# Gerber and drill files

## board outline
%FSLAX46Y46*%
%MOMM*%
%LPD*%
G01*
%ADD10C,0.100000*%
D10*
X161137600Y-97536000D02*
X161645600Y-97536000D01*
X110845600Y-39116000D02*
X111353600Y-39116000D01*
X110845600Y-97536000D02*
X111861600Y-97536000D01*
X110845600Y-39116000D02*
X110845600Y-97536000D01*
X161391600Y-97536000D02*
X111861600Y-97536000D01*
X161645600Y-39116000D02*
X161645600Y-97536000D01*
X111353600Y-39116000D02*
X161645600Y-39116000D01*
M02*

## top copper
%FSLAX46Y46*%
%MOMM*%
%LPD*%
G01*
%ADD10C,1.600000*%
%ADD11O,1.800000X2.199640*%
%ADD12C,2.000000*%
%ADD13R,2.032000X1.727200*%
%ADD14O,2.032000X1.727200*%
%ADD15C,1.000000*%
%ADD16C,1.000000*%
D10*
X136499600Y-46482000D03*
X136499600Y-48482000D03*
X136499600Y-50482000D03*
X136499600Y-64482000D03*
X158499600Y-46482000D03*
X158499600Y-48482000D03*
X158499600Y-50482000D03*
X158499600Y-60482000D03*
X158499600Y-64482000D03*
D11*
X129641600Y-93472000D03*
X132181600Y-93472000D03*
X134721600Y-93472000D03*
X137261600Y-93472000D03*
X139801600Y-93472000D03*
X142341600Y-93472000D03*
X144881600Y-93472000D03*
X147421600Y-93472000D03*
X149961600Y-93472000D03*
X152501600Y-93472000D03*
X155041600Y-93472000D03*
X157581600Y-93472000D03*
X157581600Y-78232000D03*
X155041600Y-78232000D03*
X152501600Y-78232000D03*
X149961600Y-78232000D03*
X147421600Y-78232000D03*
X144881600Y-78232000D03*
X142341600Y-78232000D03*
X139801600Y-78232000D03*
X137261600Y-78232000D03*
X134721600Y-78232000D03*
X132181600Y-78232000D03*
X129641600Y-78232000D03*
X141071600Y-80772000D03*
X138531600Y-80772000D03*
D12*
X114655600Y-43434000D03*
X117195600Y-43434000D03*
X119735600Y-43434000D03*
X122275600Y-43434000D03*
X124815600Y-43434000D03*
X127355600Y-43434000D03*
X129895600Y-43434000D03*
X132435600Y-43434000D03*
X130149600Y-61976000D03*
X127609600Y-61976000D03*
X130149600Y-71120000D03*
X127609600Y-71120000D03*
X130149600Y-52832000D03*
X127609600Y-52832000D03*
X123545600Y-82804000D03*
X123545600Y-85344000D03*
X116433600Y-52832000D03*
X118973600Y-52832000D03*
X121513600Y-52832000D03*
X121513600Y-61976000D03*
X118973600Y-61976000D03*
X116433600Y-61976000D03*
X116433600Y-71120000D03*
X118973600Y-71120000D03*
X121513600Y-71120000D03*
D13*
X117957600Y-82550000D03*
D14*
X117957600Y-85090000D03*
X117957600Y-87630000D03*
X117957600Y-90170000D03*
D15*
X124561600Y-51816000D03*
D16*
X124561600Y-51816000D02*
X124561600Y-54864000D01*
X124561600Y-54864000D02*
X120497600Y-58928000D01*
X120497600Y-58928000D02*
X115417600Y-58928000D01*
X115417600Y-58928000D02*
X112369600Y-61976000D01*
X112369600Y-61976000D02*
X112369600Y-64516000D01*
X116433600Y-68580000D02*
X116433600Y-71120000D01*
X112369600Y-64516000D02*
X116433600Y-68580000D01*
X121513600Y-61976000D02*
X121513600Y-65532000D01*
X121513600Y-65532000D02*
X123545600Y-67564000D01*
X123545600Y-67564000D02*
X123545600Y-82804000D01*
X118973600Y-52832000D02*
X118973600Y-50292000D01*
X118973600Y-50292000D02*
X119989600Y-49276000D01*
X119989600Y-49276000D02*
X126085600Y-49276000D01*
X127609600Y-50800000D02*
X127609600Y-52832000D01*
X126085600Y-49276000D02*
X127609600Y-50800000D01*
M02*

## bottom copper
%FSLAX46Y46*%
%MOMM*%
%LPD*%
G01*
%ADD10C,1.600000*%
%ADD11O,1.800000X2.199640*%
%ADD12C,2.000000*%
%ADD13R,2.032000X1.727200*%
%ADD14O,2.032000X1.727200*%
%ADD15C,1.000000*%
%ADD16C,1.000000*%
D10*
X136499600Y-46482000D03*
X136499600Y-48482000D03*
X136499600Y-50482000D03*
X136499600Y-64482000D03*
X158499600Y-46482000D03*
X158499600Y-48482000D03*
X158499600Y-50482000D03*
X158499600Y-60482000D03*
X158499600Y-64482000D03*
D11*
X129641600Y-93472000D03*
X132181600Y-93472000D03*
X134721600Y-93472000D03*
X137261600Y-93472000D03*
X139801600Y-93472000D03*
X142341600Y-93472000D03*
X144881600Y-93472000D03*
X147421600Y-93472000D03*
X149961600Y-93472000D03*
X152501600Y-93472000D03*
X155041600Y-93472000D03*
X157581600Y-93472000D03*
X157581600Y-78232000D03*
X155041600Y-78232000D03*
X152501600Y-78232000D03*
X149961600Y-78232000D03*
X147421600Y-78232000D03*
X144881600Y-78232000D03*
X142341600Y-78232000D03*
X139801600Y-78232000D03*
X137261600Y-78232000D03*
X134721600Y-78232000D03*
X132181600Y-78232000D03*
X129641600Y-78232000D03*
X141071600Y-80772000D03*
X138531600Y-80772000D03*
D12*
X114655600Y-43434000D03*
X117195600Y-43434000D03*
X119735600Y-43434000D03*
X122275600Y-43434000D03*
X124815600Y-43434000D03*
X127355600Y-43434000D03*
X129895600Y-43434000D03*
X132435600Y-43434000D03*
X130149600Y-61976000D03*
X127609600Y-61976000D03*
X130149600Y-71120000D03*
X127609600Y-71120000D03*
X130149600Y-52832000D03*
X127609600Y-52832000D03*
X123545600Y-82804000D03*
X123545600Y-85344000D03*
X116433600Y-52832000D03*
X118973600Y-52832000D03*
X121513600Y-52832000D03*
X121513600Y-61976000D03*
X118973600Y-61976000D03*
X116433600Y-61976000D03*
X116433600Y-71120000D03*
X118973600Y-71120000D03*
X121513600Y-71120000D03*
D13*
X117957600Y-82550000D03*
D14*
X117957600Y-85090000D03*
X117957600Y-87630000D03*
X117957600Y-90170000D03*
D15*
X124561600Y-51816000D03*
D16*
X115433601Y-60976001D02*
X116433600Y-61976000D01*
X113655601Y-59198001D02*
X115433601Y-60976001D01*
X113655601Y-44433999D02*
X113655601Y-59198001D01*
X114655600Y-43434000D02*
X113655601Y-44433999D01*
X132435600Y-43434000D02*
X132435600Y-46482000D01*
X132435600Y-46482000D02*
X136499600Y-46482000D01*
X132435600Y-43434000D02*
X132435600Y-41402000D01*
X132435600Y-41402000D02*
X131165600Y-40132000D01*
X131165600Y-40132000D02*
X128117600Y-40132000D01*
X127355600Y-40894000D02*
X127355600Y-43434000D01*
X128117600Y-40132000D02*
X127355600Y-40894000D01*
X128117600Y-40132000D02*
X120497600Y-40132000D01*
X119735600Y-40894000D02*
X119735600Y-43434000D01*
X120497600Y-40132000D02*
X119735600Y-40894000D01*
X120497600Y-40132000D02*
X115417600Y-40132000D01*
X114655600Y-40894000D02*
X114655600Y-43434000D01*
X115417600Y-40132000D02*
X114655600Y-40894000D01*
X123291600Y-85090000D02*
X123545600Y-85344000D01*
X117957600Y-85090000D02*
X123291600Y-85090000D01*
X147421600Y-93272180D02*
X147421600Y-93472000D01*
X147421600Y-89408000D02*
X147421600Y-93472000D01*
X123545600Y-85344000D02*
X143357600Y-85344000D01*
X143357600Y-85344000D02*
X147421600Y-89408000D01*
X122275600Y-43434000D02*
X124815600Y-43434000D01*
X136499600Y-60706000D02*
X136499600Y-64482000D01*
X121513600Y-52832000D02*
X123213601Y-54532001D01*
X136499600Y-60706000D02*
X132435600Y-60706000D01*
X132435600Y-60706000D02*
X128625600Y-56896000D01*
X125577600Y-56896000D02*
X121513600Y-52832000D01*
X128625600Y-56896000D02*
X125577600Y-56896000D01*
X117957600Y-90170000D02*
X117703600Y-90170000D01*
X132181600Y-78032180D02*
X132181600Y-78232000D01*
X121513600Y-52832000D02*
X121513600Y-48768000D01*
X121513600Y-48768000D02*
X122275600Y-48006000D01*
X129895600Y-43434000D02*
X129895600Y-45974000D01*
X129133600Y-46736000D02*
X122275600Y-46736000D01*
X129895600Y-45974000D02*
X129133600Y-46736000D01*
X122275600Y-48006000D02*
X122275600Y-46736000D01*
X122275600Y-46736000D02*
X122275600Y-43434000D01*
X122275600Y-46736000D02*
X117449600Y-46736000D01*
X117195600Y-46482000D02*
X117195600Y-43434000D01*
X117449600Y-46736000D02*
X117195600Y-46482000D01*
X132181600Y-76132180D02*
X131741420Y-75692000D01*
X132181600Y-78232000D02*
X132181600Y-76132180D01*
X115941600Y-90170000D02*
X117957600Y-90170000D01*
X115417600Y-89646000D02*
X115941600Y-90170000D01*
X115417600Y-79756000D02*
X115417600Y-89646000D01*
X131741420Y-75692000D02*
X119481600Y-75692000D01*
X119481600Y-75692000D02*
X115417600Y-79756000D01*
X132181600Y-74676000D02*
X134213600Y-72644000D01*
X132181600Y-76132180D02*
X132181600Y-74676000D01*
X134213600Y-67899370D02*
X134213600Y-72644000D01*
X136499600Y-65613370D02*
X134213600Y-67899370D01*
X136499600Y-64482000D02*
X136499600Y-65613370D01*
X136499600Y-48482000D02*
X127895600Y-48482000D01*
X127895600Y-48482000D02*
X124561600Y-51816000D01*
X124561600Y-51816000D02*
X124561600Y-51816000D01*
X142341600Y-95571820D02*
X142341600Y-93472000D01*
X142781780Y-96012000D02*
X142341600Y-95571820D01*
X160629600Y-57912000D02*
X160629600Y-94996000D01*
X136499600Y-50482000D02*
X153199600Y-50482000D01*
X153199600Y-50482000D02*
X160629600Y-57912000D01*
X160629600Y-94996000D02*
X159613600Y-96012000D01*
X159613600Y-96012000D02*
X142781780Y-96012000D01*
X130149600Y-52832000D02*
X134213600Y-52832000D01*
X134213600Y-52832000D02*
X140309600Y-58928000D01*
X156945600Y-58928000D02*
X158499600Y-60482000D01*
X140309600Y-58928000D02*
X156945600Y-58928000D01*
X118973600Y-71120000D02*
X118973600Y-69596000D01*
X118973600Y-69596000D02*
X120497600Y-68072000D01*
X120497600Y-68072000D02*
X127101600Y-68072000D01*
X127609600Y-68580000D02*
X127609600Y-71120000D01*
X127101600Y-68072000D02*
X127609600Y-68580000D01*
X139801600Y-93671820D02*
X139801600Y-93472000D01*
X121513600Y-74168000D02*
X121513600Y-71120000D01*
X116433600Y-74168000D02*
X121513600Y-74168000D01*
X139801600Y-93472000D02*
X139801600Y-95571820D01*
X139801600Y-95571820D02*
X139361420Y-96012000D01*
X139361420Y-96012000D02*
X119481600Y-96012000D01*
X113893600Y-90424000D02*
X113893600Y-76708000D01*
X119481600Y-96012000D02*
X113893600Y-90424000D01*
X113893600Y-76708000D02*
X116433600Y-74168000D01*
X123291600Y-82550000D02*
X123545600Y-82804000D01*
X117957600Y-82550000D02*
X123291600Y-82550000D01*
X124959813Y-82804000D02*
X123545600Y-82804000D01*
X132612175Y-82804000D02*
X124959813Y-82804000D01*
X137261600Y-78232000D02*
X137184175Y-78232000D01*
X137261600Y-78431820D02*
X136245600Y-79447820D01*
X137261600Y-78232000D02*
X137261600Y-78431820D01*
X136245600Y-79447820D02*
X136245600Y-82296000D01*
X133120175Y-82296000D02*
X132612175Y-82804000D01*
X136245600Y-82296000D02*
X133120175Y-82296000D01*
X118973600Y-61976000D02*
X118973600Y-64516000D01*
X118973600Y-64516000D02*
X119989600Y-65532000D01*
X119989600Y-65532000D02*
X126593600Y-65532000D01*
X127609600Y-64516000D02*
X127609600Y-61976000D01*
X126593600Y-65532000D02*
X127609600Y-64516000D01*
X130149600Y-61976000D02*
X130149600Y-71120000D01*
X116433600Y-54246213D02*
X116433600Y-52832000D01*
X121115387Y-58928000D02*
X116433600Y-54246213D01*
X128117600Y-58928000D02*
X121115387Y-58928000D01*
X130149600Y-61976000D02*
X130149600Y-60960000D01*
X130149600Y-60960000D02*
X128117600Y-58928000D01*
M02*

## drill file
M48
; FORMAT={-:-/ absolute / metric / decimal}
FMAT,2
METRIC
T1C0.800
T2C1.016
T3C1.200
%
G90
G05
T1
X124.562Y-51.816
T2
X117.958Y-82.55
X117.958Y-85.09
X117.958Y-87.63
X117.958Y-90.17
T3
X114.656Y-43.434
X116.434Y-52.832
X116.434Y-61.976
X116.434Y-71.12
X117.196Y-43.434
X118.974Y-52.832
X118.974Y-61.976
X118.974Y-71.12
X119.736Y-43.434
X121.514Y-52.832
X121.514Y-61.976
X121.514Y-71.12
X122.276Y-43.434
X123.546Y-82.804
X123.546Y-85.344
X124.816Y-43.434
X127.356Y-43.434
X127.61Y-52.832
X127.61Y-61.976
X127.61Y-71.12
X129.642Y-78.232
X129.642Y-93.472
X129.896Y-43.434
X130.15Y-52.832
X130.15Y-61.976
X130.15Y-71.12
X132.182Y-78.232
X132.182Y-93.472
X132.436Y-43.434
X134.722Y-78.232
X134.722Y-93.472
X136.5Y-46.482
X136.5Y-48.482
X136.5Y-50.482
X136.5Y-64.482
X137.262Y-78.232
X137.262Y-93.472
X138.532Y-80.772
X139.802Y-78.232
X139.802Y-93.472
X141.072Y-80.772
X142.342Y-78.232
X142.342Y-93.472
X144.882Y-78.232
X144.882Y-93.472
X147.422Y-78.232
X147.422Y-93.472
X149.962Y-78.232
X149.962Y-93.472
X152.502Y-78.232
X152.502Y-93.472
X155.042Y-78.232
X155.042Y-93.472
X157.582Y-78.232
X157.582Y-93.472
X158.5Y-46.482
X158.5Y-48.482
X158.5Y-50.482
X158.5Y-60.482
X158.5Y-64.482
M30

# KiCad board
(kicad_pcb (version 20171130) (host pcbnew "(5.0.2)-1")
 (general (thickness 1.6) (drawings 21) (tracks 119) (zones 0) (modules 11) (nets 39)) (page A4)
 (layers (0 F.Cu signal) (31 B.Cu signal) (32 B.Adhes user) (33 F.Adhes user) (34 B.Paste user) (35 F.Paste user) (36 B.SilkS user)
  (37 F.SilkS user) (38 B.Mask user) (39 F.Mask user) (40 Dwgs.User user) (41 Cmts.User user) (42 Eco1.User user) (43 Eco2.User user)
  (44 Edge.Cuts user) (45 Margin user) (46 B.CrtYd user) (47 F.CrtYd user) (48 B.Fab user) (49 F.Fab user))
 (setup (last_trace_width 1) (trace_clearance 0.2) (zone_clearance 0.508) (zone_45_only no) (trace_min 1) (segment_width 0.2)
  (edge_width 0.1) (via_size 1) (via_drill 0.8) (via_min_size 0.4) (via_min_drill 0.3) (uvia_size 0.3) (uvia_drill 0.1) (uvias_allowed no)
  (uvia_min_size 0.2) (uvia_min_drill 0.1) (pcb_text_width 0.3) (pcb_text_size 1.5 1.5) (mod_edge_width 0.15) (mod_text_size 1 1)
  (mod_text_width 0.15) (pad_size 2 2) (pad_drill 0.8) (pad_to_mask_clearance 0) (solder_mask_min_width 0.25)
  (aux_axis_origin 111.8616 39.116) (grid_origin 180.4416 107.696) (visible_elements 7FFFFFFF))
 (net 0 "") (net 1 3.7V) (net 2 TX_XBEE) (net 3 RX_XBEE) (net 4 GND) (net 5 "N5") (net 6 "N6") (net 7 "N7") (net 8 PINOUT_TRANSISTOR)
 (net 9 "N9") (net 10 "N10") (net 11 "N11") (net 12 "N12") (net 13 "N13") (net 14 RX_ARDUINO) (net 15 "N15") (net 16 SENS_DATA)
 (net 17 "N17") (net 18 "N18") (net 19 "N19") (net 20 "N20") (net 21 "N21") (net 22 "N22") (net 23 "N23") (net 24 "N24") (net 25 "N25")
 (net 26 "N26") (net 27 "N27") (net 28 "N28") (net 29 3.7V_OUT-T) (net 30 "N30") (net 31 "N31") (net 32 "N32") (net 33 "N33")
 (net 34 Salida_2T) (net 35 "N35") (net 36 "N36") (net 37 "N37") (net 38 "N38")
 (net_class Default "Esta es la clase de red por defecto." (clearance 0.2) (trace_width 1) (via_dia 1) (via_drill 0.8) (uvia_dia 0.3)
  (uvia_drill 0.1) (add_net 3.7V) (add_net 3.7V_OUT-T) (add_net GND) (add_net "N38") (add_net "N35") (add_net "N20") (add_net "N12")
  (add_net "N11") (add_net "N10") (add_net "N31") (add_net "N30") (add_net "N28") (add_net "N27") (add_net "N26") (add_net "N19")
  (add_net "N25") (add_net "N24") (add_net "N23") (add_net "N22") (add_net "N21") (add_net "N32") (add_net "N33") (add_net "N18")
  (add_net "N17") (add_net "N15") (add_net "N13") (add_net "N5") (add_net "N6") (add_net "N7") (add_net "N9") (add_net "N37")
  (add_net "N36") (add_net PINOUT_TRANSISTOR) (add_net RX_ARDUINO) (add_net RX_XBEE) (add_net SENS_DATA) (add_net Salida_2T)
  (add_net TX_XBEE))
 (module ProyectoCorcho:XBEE (layer F.Cu) (at 135.2296 45.212)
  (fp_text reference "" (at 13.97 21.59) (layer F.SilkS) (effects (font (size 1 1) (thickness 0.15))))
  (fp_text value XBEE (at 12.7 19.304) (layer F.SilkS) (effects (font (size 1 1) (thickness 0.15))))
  (pad 1 thru_hole circle (at 1.27 1.27) (size 1.6 1.6) (drill 1.2) (layers *.Cu *.Mask) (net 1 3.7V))
  (pad 2 thru_hole circle (at 1.27 3.27) (size 1.6 1.6) (drill 1.2) (layers *.Cu *.Mask) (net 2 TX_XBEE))
  (pad 3 thru_hole circle (at 1.27 5.27) (size 1.6 1.6) (drill 1.2) (layers *.Cu *.Mask) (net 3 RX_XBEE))
  (pad 4 thru_hole circle (at 1.27 19.27) (size 1.6 1.6) (drill 1.2) (layers *.Cu *.Mask) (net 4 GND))
  (pad 5 thru_hole circle (at 23.27 1.27) (size 1.6 1.6) (drill 1.2) (layers *.Cu *.Mask) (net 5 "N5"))
  (pad 6 thru_hole circle (at 23.27 3.27) (size 1.6 1.6) (drill 1.2) (layers *.Cu *.Mask) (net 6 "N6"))
  (pad 7 thru_hole circle (at 23.27 5.27) (size 1.6 1.6) (drill 1.2) (layers *.Cu *.Mask) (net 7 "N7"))
  (pad 8 thru_hole circle (at 23.27 15.27) (size 1.6 1.6) (drill 1.2) (layers *.Cu *.Mask) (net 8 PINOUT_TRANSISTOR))
  (pad 9 thru_hole circle (at 23.27 19.27) (size 1.6 1.6) (drill 1.2) (layers *.Cu *.Mask) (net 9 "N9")))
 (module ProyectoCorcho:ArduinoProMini (layer F.Cu) (at 143.6116 85.852)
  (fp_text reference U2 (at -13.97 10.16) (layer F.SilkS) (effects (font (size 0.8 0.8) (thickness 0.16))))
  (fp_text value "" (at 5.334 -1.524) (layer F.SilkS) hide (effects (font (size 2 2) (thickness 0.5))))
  (pad 12 thru_hole oval (at -13.97 7.62) (size 1.8 2.19964) (drill 1.2) (layers *.Cu *.Mask) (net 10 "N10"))
  (pad 11 thru_hole oval (at -11.43 7.62) (size 1.8 2.19964) (drill 1.2) (layers *.Cu *.Mask) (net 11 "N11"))
  (pad 10 thru_hole oval (at -8.89 7.62) (size 1.8 2.19964) (drill 1.2) (layers *.Cu *.Mask) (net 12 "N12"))
  (pad 9 thru_hole oval (at -6.35 7.62) (size 1.8 2.19964) (drill 1.2) (layers *.Cu *.Mask) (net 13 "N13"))
  (pad 8 thru_hole oval (at -3.81 7.62) (size 1.8 2.19964) (drill 1.2) (layers *.Cu *.Mask) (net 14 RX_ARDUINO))
  (pad 7 thru_hole oval (at -1.27 7.62) (size 1.8 2.19964) (drill 1.2) (layers *.Cu *.Mask) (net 3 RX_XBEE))
  (pad 6 thru_hole oval (at 1.27 7.62) (size 1.8 2.19964) (drill 1.2) (layers *.Cu *.Mask) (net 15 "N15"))
  (pad 5 thru_hole oval (at 3.81 7.62) (size 1.8 2.19964) (drill 1.2) (layers *.Cu *.Mask) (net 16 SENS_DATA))
  (pad 4 thru_hole oval (at 6.35 7.62) (size 1.8 2.19964) (drill 1.2) (layers *.Cu *.Mask) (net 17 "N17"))
  (pad 3 thru_hole oval (at 8.89 7.62) (size 1.8 2.19964) (drill 1.2) (layers *.Cu *.Mask) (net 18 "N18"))
  (pad 2 thru_hole oval (at 11.43 7.62) (size 1.8 2.19964) (drill 1.2) (layers *.Cu *.Mask) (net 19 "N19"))
  (pad 1 thru_hole oval (at 13.97 7.62) (size 1.8 2.19964) (drill 1.2) (layers *.Cu *.Mask) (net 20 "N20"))
  (pad 24 thru_hole oval (at 13.97 -7.62) (size 1.8 2.19964) (drill 1.2) (layers *.Cu *.Mask) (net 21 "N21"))
  (pad 23 thru_hole oval (at 11.43 -7.62) (size 1.8 2.19964) (drill 1.2) (layers *.Cu *.Mask) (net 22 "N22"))
  (pad 22 thru_hole oval (at 8.89 -7.62) (size 1.8 2.19964) (drill 1.2) (layers *.Cu *.Mask) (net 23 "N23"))
  (pad 21 thru_hole oval (at 6.35 -7.62) (size 1.8 2.19964) (drill 1.2) (layers *.Cu *.Mask) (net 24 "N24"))
  (pad 20 thru_hole oval (at 3.81 -7.62) (size 1.8 2.19964) (drill 1.2) (layers *.Cu *.Mask) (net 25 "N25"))
  (pad 19 thru_hole oval (at 1.27 -7.62) (size 1.8 2.19964) (drill 1.2) (layers *.Cu *.Mask) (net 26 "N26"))
  (pad 18 thru_hole oval (at -1.27 -7.62) (size 1.8 2.19964) (drill 1.2) (layers *.Cu *.Mask) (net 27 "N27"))
  (pad 17 thru_hole oval (at -3.81 -7.62) (size 1.8 2.19964) (drill 1.2) (layers *.Cu *.Mask) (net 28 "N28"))
  (pad 16 thru_hole oval (at -6.35 -7.62) (size 1.8 2.19964) (drill 1.2) (layers *.Cu *.Mask) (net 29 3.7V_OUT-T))
  (pad 15 thru_hole oval (at -8.89 -7.62) (size 1.8 2.19964) (drill 1.2) (layers *.Cu *.Mask) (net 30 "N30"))
  (pad 14 thru_hole oval (at -11.43 -7.62) (size 1.8 2.19964) (drill 1.2) (layers *.Cu *.Mask) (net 4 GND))
  (pad 13 thru_hole oval (at -13.97 -7.62) (size 1.8 2.19964) (drill 1.2) (layers *.Cu *.Mask) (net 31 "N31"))
  (pad 25 thru_hole oval (at -2.54 -5.08) (size 1.8 2.19964) (drill 1.2) (layers *.Cu *.Mask) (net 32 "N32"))
  (pad 26 thru_hole oval (at -5.08 -5.08) (size 1.8 2.19964) (drill 1.2) (layers *.Cu *.Mask) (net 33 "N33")))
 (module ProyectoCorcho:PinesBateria (layer F.Cu) (at 113.3856 42.164)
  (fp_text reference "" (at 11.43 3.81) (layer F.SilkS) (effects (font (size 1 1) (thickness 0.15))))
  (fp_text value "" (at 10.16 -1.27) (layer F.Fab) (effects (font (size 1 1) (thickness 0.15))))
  (pad 1 thru_hole circle (at 1.27 1.27) (size 2 2) (drill 1.2) (layers *.Cu *.Mask) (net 1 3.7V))
  (pad 2 thru_hole circle (at 3.81 1.27) (size 2 2) (drill 1.2) (layers *.Cu *.Mask) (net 4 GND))
  (pad 3 thru_hole circle (at 6.35 1.27) (size 2 2) (drill 1.2) (layers *.Cu *.Mask) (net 1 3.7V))
  (pad 4 thru_hole circle (at 8.89 1.27) (size 2 2) (drill 1.2) (layers *.Cu *.Mask) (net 4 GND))
  (pad 5 thru_hole circle (at 11.43 1.27) (size 2 2) (drill 1.2) (layers *.Cu *.Mask) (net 4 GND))
  (pad 6 thru_hole circle (at 13.97 1.27) (size 2 2) (drill 1.2) (layers *.Cu *.Mask) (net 1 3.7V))
  (pad 7 thru_hole circle (at 16.51 1.27) (size 2 2) (drill 1.2) (layers *.Cu *.Mask) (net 4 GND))
  (pad 8 thru_hole circle (at 19.05 1.27) (size 2 2) (drill 1.2) (layers *.Cu *.Mask) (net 1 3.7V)))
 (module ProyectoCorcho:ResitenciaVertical (layer F.Cu) (at 127.6096 61.976)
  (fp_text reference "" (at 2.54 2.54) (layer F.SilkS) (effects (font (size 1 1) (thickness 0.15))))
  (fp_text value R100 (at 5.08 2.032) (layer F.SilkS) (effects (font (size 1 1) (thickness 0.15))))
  (pad 2 thru_hole circle (at 2.54 0) (size 2 2) (drill 1.2) (layers *.Cu *.Mask) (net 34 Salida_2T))
  (pad 1 thru_hole circle (at 0 0) (size 2 2) (drill 1.2) (layers *.Cu *.Mask) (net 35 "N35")))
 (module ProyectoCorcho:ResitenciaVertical (layer F.Cu) (at 127.6096 71.12)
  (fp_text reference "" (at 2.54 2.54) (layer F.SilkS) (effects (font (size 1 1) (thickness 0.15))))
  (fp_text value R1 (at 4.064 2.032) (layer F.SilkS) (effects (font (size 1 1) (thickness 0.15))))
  (pad 2 thru_hole circle (at 2.54 0) (size 2 2) (drill 1.2) (layers *.Cu *.Mask) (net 34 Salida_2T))
  (pad 1 thru_hole circle (at 0 0) (size 2 2) (drill 1.2) (layers *.Cu *.Mask) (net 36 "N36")))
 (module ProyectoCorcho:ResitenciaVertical (layer F.Cu) (at 127.6096 52.832)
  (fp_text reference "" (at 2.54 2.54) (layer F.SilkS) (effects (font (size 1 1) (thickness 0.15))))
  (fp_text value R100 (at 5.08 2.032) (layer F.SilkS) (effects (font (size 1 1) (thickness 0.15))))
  (pad 2 thru_hole circle (at 2.54 0) (size 2 2) (drill 1.2) (layers *.Cu *.Mask) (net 8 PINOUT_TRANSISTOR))
  (pad 1 thru_hole circle (at 0 0) (size 2 2) (drill 1.2) (layers *.Cu *.Mask) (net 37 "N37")))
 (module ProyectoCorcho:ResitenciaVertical (layer F.Cu) (at 123.5456 82.804 270)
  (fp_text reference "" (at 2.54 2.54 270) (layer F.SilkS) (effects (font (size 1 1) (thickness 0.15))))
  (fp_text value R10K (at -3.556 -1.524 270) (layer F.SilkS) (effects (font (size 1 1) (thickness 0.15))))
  (pad 1 thru_hole circle (at 0 0 270) (size 2 2) (drill 1.2) (layers *.Cu *.Mask) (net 29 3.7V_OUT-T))
  (pad 2 thru_hole circle (at 2.54 0 270) (size 2 2) (drill 1.2) (layers *.Cu *.Mask) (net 16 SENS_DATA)))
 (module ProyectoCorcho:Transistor (layer F.Cu) (at 118.9736 52.832)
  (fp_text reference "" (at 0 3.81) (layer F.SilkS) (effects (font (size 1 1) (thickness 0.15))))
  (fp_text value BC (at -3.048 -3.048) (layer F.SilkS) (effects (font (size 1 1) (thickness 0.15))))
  (pad 1 thru_hole circle (at -2.54 0) (size 2 2) (drill 1.2) (layers *.Cu *.Mask) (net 34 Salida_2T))
  (pad 2 thru_hole circle (at 0 0) (size 2 2) (drill 1.2) (layers *.Cu *.Mask) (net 37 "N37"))
  (pad 3 thru_hole circle (at 2.54 0) (size 2 2) (drill 1.2) (layers *.Cu *.Mask) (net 4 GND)))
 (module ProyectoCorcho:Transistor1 (layer B.Cu) (at 118.9736 61.976)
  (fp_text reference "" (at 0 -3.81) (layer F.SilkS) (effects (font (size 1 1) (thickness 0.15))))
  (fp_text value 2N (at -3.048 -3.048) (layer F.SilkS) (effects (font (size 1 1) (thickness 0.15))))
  (pad 3 thru_hole circle (at 2.54 0) (size 2 2) (drill 1.2) (layers *.Cu *.Mask) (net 29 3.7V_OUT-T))
  (pad 2 thru_hole circle (at 0 0) (size 2 2) (drill 1.2) (layers *.Cu *.Mask) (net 35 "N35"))
  (pad 1 thru_hole circle (at -2.54 0) (size 2 2) (drill 1.2) (layers *.Cu *.Mask) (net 1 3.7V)))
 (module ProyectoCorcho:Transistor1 (layer F.Cu) (at 118.9736 71.12)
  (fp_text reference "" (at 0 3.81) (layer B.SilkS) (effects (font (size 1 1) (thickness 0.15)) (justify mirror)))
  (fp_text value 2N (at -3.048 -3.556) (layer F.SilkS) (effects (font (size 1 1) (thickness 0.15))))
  (pad 1 thru_hole circle (at -2.54 0) (size 2 2) (drill 1.2) (layers *.Cu *.Mask) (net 2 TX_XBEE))
  (pad 2 thru_hole circle (at 0 0) (size 2 2) (drill 1.2) (layers *.Cu *.Mask) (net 36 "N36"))
  (pad 3 thru_hole circle (at 2.54 0) (size 2 2) (drill 1.2) (layers *.Cu *.Mask) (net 14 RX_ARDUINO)))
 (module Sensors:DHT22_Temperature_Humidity (layer F.Cu) (at 117.9576 86.36 270)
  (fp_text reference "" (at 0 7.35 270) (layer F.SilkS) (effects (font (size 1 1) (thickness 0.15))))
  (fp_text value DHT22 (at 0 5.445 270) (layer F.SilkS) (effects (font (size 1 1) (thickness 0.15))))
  (pad 1 thru_hole rect (at -3.81 0) (size 2.032 1.7272) (drill 1.016) (layers *.Cu *.Mask F.SilkS) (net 29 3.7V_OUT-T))
  (pad 2 thru_hole oval (at -1.27 0) (size 2.032 1.7272) (drill 1.016) (layers *.Cu *.Mask F.SilkS) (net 16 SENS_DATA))
  (pad 3 thru_hole oval (at 1.27 0) (size 2.032 1.7272) (drill 1.016) (layers *.Cu *.Mask F.SilkS) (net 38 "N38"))
  (pad 4 thru_hole oval (at 3.81 0) (size 2.032 1.7272) (drill 1.016) (layers *.Cu *.Mask F.SilkS) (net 4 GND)))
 (gr_line (start 161.1376 97.536) (end 161.6456 97.536) (layer Edge.Cuts) (width 0.1))
 (gr_line (start 110.8456 39.116) (end 111.3536 39.116) (layer Edge.Cuts) (width 0.1))
 (gr_line (start 110.8456 97.536) (end 111.8616 97.536) (layer Edge.Cuts) (width 0.1))
 (gr_line (start 110.8456 39.116) (end 110.8456 97.536) (layer Edge.Cuts) (width 0.1))
 (gr_line (start 161.3916 97.536) (end 111.8616 97.536) (layer Edge.Cuts) (width 0.1))
 (gr_line (start 161.6456 39.116) (end 161.6456 97.536) (layer Edge.Cuts) (width 0.1))
 (gr_line (start 111.3536 39.116) (end 161.6456 39.116) (layer Edge.Cuts) (width 0.1))
 (segment (start 115.433601 60.976001) (end 116.4336 61.976) (width 1) (layer B.Cu) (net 1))
 (segment (start 113.655601 59.198001) (end 115.433601 60.976001) (width 1) (layer B.Cu) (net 1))
 (segment (start 113.655601 44.433999) (end 113.655601 59.198001) (width 1) (layer B.Cu) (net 1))
 (segment (start 114.6556 43.434) (end 113.655601 44.433999) (width 1) (layer B.Cu) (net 1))
 (segment (start 132.4356 43.434) (end 132.4356 46.482) (width 1) (layer B.Cu) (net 1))
 (segment (start 132.4356 46.482) (end 136.4996 46.482) (width 1) (layer B.Cu) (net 1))
 (segment (start 132.4356 43.434) (end 132.4356 41.402) (width 1) (layer B.Cu) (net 1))
 (segment (start 132.4356 41.402) (end 131.1656 40.132) (width 1) (layer B.Cu) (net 1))
 (segment (start 131.1656 40.132) (end 128.1176 40.132) (width 1) (layer B.Cu) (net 1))
 (segment (start 127.3556 40.894) (end 127.3556 43.434) (width 1) (layer B.Cu) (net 1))
 (segment (start 128.1176 40.132) (end 127.3556 40.894) (width 1) (layer B.Cu) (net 1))
 (segment (start 128.1176 40.132) (end 120.4976 40.132) (width 1) (layer B.Cu) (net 1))
 (segment (start 119.7356 40.894) (end 119.7356 43.434) (width 1) (layer B.Cu) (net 1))
 (segment (start 120.4976 40.132) (end 119.7356 40.894) (width 1) (layer B.Cu) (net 1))
 (segment (start 120.4976 40.132) (end 115.4176 40.132) (width 1) (layer B.Cu) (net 1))
 (segment (start 114.6556 40.894) (end 114.6556 43.434) (width 1) (layer B.Cu) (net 1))
 (segment (start 115.4176 40.132) (end 114.6556 40.894) (width 1) (layer B.Cu) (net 1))
 (segment (start 123.2916 85.09) (end 123.5456 85.344) (width 1) (layer B.Cu) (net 16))
 (segment (start 117.9576 85.09) (end 123.2916 85.09) (width 1) (layer B.Cu) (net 16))
 (segment (start 147.4216 93.27218) (end 147.4216 93.472) (width 1) (layer B.Cu) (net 16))
 (segment (start 147.4216 89.408) (end 147.4216 93.472) (width 1) (layer B.Cu) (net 16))
 (segment (start 123.5456 85.344) (end 143.3576 85.344) (width 1) (layer B.Cu) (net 16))
 (segment (start 143.3576 85.344) (end 147.4216 89.408) (width 1) (layer B.Cu) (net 16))
 (segment (start 122.2756 43.434) (end 124.8156 43.434) (width 1) (layer B.Cu) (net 4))
 (segment (start 136.4996 60.706) (end 136.4996 64.482) (width 1) (layer B.Cu) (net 4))
 (segment (start 121.5136 52.832) (end 123.213601 54.532001) (width 1) (layer B.Cu) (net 4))
 (segment (start 136.4996 60.706) (end 132.4356 60.706) (width 1) (layer B.Cu) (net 4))
 (segment (start 132.4356 60.706) (end 128.6256 56.896) (width 1) (layer B.Cu) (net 4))
 (segment (start 125.5776 56.896) (end 121.5136 52.832) (width 1) (layer B.Cu) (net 4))
 (segment (start 128.6256 56.896) (end 125.5776 56.896) (width 1) (layer B.Cu) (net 4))
 (segment (start 117.9576 90.17) (end 117.7036 90.17) (width 1) (layer B.Cu) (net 4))
 (segment (start 132.1816 78.03218) (end 132.1816 78.232) (width 1) (layer B.Cu) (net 4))
 (segment (start 121.5136 52.832) (end 121.5136 48.768) (width 1) (layer B.Cu) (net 4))
 (segment (start 121.5136 48.768) (end 122.2756 48.006) (width 1) (layer B.Cu) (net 4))
 (segment (start 129.8956 43.434) (end 129.8956 45.974) (width 1) (layer B.Cu) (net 4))
 (segment (start 129.1336 46.736) (end 122.2756 46.736) (width 1) (layer B.Cu) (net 4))
 (segment (start 129.8956 45.974) (end 129.1336 46.736) (width 1) (layer B.Cu) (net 4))
 (segment (start 122.2756 48.006) (end 122.2756 46.736) (width 1) (layer B.Cu) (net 4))
 (segment (start 122.2756 46.736) (end 122.2756 43.434) (width 1) (layer B.Cu) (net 4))
 (segment (start 122.2756 46.736) (end 117.4496 46.736) (width 1) (layer B.Cu) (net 4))
 (segment (start 117.1956 46.482) (end 117.1956 43.434) (width 1) (layer B.Cu) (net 4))
 (segment (start 117.4496 46.736) (end 117.1956 46.482) (width 1) (layer B.Cu) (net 4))
 (segment (start 132.1816 76.13218) (end 131.74142 75.692) (width 1) (layer B.Cu) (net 4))
 (segment (start 132.1816 78.232) (end 132.1816 76.13218) (width 1) (layer B.Cu) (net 4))
 (segment (start 115.9416 90.17) (end 117.9576 90.17) (width 1) (layer B.Cu) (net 4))
 (segment (start 115.4176 89.646) (end 115.9416 90.17) (width 1) (layer B.Cu) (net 4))
 (segment (start 115.4176 79.756) (end 115.4176 89.646) (width 1) (layer B.Cu) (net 4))
 (segment (start 131.74142 75.692) (end 119.4816 75.692) (width 1) (layer B.Cu) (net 4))
 (segment (start 119.4816 75.692) (end 115.4176 79.756) (width 1) (layer B.Cu) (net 4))
 (segment (start 132.1816 74.676) (end 134.2136 72.644) (width 1) (layer B.Cu) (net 4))
 (segment (start 132.1816 76.13218) (end 132.1816 74.676) (width 1) (layer B.Cu) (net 4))
 (segment (start 134.2136 67.89937) (end 134.2136 72.644) (width 1) (layer B.Cu) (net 4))
 (segment (start 136.4996 65.61337) (end 134.2136 67.89937) (width 1) (layer B.Cu) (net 4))
 (segment (start 136.4996 64.482) (end 136.4996 65.61337) (width 1) (layer B.Cu) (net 4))
 (segment (start 136.4996 48.482) (end 127.8956 48.482) (width 1) (layer B.Cu) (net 2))
 (segment (start 127.8956 48.482) (end 124.5616 51.816) (width 1) (layer B.Cu) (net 2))
 (segment (start 124.5616 51.816) (end 124.5616 51.816) (width 1) (layer B.Cu) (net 2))
 (via (at 124.5616 51.816) (size 1) (drill 0.8) (layers F.Cu B.Cu) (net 2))
 (segment (start 124.5616 51.816) (end 124.5616 54.864) (width 1) (layer F.Cu) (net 2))
 (segment (start 124.5616 54.864) (end 120.4976 58.928) (width 1) (layer F.Cu) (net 2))
 (segment (start 120.4976 58.928) (end 115.4176 58.928) (width 1) (layer F.Cu) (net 2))
 (segment (start 115.4176 58.928) (end 112.3696 61.976) (width 1) (layer F.Cu) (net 2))
 (segment (start 112.3696 61.976) (end 112.3696 64.516) (width 1) (layer F.Cu) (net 2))
 (segment (start 116.4336 68.58) (end 116.4336 71.12) (width 1) (layer F.Cu) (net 2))
 (segment (start 112.3696 64.516) (end 116.4336 68.58) (width 1) (layer F.Cu) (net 2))
 (segment (start 142.3416 95.57182) (end 142.3416 93.472) (width 1) (layer B.Cu) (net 3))
 (segment (start 142.78178 96.012) (end 142.3416 95.57182) (width 1) (layer B.Cu) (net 3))
 (segment (start 160.6296 57.912) (end 160.6296 94.996) (width 1) (layer B.Cu) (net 3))
 (segment (start 136.4996 50.482) (end 153.1996 50.482) (width 1) (layer B.Cu) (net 3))
 (segment (start 153.1996 50.482) (end 160.6296 57.912) (width 1) (layer B.Cu) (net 3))
 (segment (start 160.6296 94.996) (end 159.6136 96.012) (width 1) (layer B.Cu) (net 3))
 (segment (start 159.6136 96.012) (end 142.78178 96.012) (width 1) (layer B.Cu) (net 3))
 (segment (start 130.1496 52.832) (end 134.2136 52.832) (width 1) (layer B.Cu) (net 8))
 (segment (start 134.2136 52.832) (end 140.3096 58.928) (width 1) (layer B.Cu) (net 8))
 (segment (start 156.9456 58.928) (end 158.4996 60.482) (width 1) (layer B.Cu) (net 8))
 (segment (start 140.3096 58.928) (end 156.9456 58.928) (width 1) (layer B.Cu) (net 8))
 (segment (start 118.9736 71.12) (end 118.9736 69.596) (width 1) (layer B.Cu) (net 36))
 (segment (start 118.9736 69.596) (end 120.4976 68.072) (width 1) (layer B.Cu) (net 36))
 (segment (start 120.4976 68.072) (end 127.1016 68.072) (width 1) (layer B.Cu) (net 36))
 (segment (start 127.6096 68.58) (end 127.6096 71.12) (width 1) (layer B.Cu) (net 36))
 (segment (start 127.1016 68.072) (end 127.6096 68.58) (width 1) (layer B.Cu) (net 36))
 (segment (start 139.8016 93.67182) (end 139.8016 93.472) (width 1) (layer B.Cu) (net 14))
 (segment (start 121.5136 74.168) (end 121.5136 71.12) (width 1) (layer B.Cu) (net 14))
 (segment (start 116.4336 74.168) (end 121.5136 74.168) (width 1) (layer B.Cu) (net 14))
 (segment (start 139.8016 93.472) (end 139.8016 95.57182) (width 1) (layer B.Cu) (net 14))
 (segment (start 139.8016 95.57182) (end 139.36142 96.012) (width 1) (layer B.Cu) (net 14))
 (segment (start 139.36142 96.012) (end 119.4816 96.012) (width 1) (layer B.Cu) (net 14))
 (segment (start 113.8936 90.424) (end 113.8936 76.708) (width 1) (layer B.Cu) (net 14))
 (segment (start 119.4816 96.012) (end 113.8936 90.424) (width 1) (layer B.Cu) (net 14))
 (segment (start 113.8936 76.708) (end 116.4336 74.168) (width 1) (layer B.Cu) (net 14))
 (segment (start 123.2916 82.55) (end 123.5456 82.804) (width 1) (layer B.Cu) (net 29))
 (segment (start 117.9576 82.55) (end 123.2916 82.55) (width 1) (layer B.Cu) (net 29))
 (segment (start 124.959813 82.804) (end 123.5456 82.804) (width 1) (layer B.Cu) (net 29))
 (segment (start 132.612175 82.804) (end 124.959813 82.804) (width 1) (layer B.Cu) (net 29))
 (segment (start 137.2616 78.232) (end 137.184175 78.232) (width 1) (layer B.Cu) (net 29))
 (segment (start 121.5136 61.976) (end 121.5136 65.532) (width 1) (layer F.Cu) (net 29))
 (segment (start 121.5136 65.532) (end 123.5456 67.564) (width 1) (layer F.Cu) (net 29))
 (segment (start 123.5456 67.564) (end 123.5456 82.804) (width 1) (layer F.Cu) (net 29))
 (segment (start 137.2616 78.43182) (end 136.2456 79.44782) (width 1) (layer B.Cu) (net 29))
 (segment (start 137.2616 78.232) (end 137.2616 78.43182) (width 1) (layer B.Cu) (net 29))
 (segment (start 136.2456 79.44782) (end 136.2456 82.296) (width 1) (layer B.Cu) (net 29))
 (segment (start 133.120175 82.296) (end 132.612175 82.804) (width 1) (layer B.Cu) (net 29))
 (segment (start 136.2456 82.296) (end 133.120175 82.296) (width 1) (layer B.Cu) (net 29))
 (segment (start 118.9736 61.976) (end 118.9736 64.516) (width 1) (layer B.Cu) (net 35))
 (segment (start 118.9736 64.516) (end 119.9896 65.532) (width 1) (layer B.Cu) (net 35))
 (segment (start 119.9896 65.532) (end 126.5936 65.532) (width 1) (layer B.Cu) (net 35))
 (segment (start 127.6096 64.516) (end 127.6096 61.976) (width 1) (layer B.Cu) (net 35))
 (segment (start 126.5936 65.532) (end 127.6096 64.516) (width 1) (layer B.Cu) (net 35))
 (segment (start 130.1496 61.976) (end 130.1496 71.12) (width 1) (layer B.Cu) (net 34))
 (segment (start 116.4336 54.246213) (end 116.4336 52.832) (width 1) (layer B.Cu) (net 34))
 (segment (start 121.115387 58.928) (end 116.4336 54.246213) (width 1) (layer B.Cu) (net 34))
 (segment (start 128.1176 58.928) (end 121.115387 58.928) (width 1) (layer B.Cu) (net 34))
 (segment (start 130.1496 61.976) (end 130.1496 60.96) (width 1) (layer B.Cu) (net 34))
 (segment (start 130.1496 60.96) (end 128.1176 58.928) (width 1) (layer B.Cu) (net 34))
 (segment (start 118.9736 52.832) (end 118.9736 50.292) (width 1) (layer F.Cu) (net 37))
 (segment (start 118.9736 50.292) (end 119.9896 49.276) (width 1) (layer F.Cu) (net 37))
 (segment (start 119.9896 49.276) (end 126.0856 49.276) (width 1) (layer F.Cu) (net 37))
 (segment (start 127.6096 50.8) (end 127.6096 52.832) (width 1) (layer F.Cu) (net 37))
 (segment (start 126.0856 49.276) (end 127.6096 50.8) (width 1) (layer F.Cu) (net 37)))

